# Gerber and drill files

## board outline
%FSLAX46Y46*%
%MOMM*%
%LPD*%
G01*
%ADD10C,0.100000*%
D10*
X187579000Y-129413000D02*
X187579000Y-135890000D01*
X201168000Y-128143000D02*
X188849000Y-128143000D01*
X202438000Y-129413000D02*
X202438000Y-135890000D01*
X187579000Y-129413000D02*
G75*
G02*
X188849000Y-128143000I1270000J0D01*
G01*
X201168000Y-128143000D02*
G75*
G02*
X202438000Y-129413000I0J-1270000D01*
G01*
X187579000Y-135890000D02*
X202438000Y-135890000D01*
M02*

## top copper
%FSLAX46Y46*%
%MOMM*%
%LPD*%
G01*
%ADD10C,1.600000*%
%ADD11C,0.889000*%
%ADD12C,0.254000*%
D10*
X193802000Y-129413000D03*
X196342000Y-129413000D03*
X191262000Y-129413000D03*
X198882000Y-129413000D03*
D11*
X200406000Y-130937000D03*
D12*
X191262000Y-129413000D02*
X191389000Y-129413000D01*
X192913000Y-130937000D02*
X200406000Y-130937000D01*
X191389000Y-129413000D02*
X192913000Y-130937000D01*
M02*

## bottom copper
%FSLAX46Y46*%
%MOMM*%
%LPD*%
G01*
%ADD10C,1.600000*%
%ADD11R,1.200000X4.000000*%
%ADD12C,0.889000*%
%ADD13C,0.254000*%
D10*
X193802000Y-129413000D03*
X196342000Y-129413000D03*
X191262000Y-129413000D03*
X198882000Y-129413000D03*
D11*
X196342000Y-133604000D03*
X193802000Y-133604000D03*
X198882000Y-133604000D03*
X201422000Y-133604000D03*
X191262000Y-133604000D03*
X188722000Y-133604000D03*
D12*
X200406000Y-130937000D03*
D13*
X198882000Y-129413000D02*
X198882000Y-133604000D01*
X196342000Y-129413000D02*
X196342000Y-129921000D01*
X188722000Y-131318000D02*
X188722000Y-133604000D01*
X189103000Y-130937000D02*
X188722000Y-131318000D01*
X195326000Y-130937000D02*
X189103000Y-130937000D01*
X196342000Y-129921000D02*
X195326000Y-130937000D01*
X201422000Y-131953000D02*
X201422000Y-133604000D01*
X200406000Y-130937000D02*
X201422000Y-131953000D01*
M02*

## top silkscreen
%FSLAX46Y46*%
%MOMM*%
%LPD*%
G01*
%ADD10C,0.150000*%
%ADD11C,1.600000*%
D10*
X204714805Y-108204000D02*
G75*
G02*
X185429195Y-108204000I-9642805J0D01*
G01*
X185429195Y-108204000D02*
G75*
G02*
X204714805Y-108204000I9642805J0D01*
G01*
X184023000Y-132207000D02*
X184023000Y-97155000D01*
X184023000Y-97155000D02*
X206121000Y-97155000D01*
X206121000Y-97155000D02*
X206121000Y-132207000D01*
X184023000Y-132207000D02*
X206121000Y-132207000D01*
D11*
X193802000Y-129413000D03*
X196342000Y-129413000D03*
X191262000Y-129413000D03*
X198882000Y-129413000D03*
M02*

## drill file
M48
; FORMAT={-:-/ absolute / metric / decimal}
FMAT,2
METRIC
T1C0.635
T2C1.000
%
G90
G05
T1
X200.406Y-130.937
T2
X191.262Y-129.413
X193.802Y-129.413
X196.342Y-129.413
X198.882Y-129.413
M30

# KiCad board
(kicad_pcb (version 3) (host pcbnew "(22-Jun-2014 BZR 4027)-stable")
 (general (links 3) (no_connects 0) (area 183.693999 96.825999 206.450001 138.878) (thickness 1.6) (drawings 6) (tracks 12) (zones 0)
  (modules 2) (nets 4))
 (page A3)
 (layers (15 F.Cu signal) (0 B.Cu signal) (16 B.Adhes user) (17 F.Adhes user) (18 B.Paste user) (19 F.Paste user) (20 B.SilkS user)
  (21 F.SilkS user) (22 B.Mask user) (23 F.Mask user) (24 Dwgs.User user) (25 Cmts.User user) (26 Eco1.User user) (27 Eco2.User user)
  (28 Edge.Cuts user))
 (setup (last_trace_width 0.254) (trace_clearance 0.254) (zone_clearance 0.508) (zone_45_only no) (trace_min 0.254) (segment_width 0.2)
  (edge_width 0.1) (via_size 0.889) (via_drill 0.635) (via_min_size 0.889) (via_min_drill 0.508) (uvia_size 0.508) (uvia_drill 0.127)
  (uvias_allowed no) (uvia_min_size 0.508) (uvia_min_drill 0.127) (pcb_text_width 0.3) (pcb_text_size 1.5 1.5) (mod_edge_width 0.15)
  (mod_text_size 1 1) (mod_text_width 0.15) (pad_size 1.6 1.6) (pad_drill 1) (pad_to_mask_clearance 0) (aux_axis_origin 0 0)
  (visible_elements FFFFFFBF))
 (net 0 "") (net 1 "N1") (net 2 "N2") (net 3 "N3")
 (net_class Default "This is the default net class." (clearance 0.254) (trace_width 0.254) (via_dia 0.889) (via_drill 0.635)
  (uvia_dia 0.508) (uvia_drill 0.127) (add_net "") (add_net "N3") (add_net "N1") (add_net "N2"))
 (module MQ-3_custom (layer F.Cu) (at 195.072 129.413)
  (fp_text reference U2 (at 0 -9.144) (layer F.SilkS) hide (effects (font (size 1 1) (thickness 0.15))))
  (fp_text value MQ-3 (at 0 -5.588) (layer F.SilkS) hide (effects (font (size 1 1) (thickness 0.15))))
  (fp_circle (center 0 -21.209) (end 7.366 -14.986) (layer F.SilkS) (width 0.15))
  (fp_line (start -11.049 2.794) (end -11.049 -32.258) (layer F.SilkS) (width 0.15))
  (fp_line (start -11.049 -32.258) (end 11.049 -32.258) (layer F.SilkS) (width 0.15))
  (fp_line (start 11.049 -32.258) (end 11.049 2.794) (layer F.SilkS) (width 0.15))
  (fp_line (start -11.049 2.794) (end 11.049 2.794) (layer F.SilkS) (width 0.15))
  (pad 2 thru_hole circle (at -1.27 0) (size 1.6 1.6) (drill 1) (layers *.Cu *.Mask F.SilkS))
  (pad 3 thru_hole circle (at 1.27 0) (size 1.6 1.6) (drill 1) (layers *.Cu *.Mask F.SilkS) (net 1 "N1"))
  (pad 1 thru_hole circle (at -3.81 0) (size 1.6 1.6) (drill 1) (layers *.Cu *.Mask F.SilkS) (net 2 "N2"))
  (pad 4 thru_hole circle (at 3.81 0) (size 1.6 1.6) (drill 1) (layers *.Cu *.Mask F.SilkS) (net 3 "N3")))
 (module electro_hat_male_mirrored (layer B.Cu) (at 195.072 133.604)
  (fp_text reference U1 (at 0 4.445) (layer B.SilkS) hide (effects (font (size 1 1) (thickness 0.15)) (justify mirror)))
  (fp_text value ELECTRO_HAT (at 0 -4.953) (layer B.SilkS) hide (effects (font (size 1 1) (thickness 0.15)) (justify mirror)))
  (pad 3 smd rect (at 1.27 0) (size 1.2 4) (layers B.Cu B.Paste B.Mask))
  (pad 4 smd rect (at -1.27 0) (size 1.2 4) (layers B.Cu B.Paste B.Mask))
  (pad 2 smd rect (at 3.81 0) (size 1.2 4) (layers B.Cu B.Paste B.Mask) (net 3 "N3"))
  (pad 1 smd rect (at 6.35 0) (size 1.2 4) (layers B.Cu B.Paste B.Mask) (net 2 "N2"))
  (pad 5 smd rect (at -3.81 0) (size 1.2 4) (layers B.Cu B.Paste B.Mask))
  (pad 6 smd rect (at -6.35 0) (size 1.2 4) (layers B.Cu B.Paste B.Mask) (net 1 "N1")))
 (gr_line (start 187.579 129.413) (end 187.579 135.89) (angle 90) (layer Edge.Cuts) (width 0.1))
 (gr_line (start 201.168 128.143) (end 188.849 128.143) (angle 90) (layer Edge.Cuts) (width 0.1))
 (gr_line (start 202.438 129.413) (end 202.438 135.89) (angle 90) (layer Edge.Cuts) (width 0.1))
 (gr_arc (start 188.849 129.413) (end 187.579 129.413) (angle 90) (layer Edge.Cuts) (width 0.1))
 (gr_arc (start 201.168 129.413) (end 201.168 128.143) (angle 90) (layer Edge.Cuts) (width 0.1))
 (gr_line (start 187.579 135.89) (end 202.438 135.89) (angle 90) (layer Edge.Cuts) (width 0.1))
 (segment (start 198.882 129.413) (end 198.882 133.604) (width 0.254) (layer B.Cu) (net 3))
 (segment (start 196.342 129.413) (end 196.342 129.921) (width 0.254) (layer B.Cu) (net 1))
 (segment (start 188.722 131.318) (end 188.722 133.604) (width 0.254) (layer B.Cu) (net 1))
 (segment (start 189.103 130.937) (end 188.722 131.318) (width 0.254) (layer B.Cu) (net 1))
 (segment (start 195.326 130.937) (end 189.103 130.937) (width 0.254) (layer B.Cu) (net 1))
 (segment (start 196.342 129.921) (end 195.326 130.937) (width 0.254) (layer B.Cu) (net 1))
 (segment (start 191.262 129.413) (end 191.389 129.413) (width 0.254) (layer F.Cu) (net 2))
 (segment (start 201.422 131.953) (end 201.422 133.604) (width 0.254) (layer B.Cu) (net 2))
 (segment (start 200.406 130.937) (end 201.422 131.953) (width 0.254) (layer B.Cu) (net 2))
 (via (at 200.406 130.937) (size 0.889) (layers F.Cu B.Cu) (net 2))
 (segment (start 192.913 130.937) (end 200.406 130.937) (width 0.254) (layer F.Cu) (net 2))
 (segment (start 191.389 129.413) (end 192.913 130.937) (width 0.254) (layer F.Cu) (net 2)))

